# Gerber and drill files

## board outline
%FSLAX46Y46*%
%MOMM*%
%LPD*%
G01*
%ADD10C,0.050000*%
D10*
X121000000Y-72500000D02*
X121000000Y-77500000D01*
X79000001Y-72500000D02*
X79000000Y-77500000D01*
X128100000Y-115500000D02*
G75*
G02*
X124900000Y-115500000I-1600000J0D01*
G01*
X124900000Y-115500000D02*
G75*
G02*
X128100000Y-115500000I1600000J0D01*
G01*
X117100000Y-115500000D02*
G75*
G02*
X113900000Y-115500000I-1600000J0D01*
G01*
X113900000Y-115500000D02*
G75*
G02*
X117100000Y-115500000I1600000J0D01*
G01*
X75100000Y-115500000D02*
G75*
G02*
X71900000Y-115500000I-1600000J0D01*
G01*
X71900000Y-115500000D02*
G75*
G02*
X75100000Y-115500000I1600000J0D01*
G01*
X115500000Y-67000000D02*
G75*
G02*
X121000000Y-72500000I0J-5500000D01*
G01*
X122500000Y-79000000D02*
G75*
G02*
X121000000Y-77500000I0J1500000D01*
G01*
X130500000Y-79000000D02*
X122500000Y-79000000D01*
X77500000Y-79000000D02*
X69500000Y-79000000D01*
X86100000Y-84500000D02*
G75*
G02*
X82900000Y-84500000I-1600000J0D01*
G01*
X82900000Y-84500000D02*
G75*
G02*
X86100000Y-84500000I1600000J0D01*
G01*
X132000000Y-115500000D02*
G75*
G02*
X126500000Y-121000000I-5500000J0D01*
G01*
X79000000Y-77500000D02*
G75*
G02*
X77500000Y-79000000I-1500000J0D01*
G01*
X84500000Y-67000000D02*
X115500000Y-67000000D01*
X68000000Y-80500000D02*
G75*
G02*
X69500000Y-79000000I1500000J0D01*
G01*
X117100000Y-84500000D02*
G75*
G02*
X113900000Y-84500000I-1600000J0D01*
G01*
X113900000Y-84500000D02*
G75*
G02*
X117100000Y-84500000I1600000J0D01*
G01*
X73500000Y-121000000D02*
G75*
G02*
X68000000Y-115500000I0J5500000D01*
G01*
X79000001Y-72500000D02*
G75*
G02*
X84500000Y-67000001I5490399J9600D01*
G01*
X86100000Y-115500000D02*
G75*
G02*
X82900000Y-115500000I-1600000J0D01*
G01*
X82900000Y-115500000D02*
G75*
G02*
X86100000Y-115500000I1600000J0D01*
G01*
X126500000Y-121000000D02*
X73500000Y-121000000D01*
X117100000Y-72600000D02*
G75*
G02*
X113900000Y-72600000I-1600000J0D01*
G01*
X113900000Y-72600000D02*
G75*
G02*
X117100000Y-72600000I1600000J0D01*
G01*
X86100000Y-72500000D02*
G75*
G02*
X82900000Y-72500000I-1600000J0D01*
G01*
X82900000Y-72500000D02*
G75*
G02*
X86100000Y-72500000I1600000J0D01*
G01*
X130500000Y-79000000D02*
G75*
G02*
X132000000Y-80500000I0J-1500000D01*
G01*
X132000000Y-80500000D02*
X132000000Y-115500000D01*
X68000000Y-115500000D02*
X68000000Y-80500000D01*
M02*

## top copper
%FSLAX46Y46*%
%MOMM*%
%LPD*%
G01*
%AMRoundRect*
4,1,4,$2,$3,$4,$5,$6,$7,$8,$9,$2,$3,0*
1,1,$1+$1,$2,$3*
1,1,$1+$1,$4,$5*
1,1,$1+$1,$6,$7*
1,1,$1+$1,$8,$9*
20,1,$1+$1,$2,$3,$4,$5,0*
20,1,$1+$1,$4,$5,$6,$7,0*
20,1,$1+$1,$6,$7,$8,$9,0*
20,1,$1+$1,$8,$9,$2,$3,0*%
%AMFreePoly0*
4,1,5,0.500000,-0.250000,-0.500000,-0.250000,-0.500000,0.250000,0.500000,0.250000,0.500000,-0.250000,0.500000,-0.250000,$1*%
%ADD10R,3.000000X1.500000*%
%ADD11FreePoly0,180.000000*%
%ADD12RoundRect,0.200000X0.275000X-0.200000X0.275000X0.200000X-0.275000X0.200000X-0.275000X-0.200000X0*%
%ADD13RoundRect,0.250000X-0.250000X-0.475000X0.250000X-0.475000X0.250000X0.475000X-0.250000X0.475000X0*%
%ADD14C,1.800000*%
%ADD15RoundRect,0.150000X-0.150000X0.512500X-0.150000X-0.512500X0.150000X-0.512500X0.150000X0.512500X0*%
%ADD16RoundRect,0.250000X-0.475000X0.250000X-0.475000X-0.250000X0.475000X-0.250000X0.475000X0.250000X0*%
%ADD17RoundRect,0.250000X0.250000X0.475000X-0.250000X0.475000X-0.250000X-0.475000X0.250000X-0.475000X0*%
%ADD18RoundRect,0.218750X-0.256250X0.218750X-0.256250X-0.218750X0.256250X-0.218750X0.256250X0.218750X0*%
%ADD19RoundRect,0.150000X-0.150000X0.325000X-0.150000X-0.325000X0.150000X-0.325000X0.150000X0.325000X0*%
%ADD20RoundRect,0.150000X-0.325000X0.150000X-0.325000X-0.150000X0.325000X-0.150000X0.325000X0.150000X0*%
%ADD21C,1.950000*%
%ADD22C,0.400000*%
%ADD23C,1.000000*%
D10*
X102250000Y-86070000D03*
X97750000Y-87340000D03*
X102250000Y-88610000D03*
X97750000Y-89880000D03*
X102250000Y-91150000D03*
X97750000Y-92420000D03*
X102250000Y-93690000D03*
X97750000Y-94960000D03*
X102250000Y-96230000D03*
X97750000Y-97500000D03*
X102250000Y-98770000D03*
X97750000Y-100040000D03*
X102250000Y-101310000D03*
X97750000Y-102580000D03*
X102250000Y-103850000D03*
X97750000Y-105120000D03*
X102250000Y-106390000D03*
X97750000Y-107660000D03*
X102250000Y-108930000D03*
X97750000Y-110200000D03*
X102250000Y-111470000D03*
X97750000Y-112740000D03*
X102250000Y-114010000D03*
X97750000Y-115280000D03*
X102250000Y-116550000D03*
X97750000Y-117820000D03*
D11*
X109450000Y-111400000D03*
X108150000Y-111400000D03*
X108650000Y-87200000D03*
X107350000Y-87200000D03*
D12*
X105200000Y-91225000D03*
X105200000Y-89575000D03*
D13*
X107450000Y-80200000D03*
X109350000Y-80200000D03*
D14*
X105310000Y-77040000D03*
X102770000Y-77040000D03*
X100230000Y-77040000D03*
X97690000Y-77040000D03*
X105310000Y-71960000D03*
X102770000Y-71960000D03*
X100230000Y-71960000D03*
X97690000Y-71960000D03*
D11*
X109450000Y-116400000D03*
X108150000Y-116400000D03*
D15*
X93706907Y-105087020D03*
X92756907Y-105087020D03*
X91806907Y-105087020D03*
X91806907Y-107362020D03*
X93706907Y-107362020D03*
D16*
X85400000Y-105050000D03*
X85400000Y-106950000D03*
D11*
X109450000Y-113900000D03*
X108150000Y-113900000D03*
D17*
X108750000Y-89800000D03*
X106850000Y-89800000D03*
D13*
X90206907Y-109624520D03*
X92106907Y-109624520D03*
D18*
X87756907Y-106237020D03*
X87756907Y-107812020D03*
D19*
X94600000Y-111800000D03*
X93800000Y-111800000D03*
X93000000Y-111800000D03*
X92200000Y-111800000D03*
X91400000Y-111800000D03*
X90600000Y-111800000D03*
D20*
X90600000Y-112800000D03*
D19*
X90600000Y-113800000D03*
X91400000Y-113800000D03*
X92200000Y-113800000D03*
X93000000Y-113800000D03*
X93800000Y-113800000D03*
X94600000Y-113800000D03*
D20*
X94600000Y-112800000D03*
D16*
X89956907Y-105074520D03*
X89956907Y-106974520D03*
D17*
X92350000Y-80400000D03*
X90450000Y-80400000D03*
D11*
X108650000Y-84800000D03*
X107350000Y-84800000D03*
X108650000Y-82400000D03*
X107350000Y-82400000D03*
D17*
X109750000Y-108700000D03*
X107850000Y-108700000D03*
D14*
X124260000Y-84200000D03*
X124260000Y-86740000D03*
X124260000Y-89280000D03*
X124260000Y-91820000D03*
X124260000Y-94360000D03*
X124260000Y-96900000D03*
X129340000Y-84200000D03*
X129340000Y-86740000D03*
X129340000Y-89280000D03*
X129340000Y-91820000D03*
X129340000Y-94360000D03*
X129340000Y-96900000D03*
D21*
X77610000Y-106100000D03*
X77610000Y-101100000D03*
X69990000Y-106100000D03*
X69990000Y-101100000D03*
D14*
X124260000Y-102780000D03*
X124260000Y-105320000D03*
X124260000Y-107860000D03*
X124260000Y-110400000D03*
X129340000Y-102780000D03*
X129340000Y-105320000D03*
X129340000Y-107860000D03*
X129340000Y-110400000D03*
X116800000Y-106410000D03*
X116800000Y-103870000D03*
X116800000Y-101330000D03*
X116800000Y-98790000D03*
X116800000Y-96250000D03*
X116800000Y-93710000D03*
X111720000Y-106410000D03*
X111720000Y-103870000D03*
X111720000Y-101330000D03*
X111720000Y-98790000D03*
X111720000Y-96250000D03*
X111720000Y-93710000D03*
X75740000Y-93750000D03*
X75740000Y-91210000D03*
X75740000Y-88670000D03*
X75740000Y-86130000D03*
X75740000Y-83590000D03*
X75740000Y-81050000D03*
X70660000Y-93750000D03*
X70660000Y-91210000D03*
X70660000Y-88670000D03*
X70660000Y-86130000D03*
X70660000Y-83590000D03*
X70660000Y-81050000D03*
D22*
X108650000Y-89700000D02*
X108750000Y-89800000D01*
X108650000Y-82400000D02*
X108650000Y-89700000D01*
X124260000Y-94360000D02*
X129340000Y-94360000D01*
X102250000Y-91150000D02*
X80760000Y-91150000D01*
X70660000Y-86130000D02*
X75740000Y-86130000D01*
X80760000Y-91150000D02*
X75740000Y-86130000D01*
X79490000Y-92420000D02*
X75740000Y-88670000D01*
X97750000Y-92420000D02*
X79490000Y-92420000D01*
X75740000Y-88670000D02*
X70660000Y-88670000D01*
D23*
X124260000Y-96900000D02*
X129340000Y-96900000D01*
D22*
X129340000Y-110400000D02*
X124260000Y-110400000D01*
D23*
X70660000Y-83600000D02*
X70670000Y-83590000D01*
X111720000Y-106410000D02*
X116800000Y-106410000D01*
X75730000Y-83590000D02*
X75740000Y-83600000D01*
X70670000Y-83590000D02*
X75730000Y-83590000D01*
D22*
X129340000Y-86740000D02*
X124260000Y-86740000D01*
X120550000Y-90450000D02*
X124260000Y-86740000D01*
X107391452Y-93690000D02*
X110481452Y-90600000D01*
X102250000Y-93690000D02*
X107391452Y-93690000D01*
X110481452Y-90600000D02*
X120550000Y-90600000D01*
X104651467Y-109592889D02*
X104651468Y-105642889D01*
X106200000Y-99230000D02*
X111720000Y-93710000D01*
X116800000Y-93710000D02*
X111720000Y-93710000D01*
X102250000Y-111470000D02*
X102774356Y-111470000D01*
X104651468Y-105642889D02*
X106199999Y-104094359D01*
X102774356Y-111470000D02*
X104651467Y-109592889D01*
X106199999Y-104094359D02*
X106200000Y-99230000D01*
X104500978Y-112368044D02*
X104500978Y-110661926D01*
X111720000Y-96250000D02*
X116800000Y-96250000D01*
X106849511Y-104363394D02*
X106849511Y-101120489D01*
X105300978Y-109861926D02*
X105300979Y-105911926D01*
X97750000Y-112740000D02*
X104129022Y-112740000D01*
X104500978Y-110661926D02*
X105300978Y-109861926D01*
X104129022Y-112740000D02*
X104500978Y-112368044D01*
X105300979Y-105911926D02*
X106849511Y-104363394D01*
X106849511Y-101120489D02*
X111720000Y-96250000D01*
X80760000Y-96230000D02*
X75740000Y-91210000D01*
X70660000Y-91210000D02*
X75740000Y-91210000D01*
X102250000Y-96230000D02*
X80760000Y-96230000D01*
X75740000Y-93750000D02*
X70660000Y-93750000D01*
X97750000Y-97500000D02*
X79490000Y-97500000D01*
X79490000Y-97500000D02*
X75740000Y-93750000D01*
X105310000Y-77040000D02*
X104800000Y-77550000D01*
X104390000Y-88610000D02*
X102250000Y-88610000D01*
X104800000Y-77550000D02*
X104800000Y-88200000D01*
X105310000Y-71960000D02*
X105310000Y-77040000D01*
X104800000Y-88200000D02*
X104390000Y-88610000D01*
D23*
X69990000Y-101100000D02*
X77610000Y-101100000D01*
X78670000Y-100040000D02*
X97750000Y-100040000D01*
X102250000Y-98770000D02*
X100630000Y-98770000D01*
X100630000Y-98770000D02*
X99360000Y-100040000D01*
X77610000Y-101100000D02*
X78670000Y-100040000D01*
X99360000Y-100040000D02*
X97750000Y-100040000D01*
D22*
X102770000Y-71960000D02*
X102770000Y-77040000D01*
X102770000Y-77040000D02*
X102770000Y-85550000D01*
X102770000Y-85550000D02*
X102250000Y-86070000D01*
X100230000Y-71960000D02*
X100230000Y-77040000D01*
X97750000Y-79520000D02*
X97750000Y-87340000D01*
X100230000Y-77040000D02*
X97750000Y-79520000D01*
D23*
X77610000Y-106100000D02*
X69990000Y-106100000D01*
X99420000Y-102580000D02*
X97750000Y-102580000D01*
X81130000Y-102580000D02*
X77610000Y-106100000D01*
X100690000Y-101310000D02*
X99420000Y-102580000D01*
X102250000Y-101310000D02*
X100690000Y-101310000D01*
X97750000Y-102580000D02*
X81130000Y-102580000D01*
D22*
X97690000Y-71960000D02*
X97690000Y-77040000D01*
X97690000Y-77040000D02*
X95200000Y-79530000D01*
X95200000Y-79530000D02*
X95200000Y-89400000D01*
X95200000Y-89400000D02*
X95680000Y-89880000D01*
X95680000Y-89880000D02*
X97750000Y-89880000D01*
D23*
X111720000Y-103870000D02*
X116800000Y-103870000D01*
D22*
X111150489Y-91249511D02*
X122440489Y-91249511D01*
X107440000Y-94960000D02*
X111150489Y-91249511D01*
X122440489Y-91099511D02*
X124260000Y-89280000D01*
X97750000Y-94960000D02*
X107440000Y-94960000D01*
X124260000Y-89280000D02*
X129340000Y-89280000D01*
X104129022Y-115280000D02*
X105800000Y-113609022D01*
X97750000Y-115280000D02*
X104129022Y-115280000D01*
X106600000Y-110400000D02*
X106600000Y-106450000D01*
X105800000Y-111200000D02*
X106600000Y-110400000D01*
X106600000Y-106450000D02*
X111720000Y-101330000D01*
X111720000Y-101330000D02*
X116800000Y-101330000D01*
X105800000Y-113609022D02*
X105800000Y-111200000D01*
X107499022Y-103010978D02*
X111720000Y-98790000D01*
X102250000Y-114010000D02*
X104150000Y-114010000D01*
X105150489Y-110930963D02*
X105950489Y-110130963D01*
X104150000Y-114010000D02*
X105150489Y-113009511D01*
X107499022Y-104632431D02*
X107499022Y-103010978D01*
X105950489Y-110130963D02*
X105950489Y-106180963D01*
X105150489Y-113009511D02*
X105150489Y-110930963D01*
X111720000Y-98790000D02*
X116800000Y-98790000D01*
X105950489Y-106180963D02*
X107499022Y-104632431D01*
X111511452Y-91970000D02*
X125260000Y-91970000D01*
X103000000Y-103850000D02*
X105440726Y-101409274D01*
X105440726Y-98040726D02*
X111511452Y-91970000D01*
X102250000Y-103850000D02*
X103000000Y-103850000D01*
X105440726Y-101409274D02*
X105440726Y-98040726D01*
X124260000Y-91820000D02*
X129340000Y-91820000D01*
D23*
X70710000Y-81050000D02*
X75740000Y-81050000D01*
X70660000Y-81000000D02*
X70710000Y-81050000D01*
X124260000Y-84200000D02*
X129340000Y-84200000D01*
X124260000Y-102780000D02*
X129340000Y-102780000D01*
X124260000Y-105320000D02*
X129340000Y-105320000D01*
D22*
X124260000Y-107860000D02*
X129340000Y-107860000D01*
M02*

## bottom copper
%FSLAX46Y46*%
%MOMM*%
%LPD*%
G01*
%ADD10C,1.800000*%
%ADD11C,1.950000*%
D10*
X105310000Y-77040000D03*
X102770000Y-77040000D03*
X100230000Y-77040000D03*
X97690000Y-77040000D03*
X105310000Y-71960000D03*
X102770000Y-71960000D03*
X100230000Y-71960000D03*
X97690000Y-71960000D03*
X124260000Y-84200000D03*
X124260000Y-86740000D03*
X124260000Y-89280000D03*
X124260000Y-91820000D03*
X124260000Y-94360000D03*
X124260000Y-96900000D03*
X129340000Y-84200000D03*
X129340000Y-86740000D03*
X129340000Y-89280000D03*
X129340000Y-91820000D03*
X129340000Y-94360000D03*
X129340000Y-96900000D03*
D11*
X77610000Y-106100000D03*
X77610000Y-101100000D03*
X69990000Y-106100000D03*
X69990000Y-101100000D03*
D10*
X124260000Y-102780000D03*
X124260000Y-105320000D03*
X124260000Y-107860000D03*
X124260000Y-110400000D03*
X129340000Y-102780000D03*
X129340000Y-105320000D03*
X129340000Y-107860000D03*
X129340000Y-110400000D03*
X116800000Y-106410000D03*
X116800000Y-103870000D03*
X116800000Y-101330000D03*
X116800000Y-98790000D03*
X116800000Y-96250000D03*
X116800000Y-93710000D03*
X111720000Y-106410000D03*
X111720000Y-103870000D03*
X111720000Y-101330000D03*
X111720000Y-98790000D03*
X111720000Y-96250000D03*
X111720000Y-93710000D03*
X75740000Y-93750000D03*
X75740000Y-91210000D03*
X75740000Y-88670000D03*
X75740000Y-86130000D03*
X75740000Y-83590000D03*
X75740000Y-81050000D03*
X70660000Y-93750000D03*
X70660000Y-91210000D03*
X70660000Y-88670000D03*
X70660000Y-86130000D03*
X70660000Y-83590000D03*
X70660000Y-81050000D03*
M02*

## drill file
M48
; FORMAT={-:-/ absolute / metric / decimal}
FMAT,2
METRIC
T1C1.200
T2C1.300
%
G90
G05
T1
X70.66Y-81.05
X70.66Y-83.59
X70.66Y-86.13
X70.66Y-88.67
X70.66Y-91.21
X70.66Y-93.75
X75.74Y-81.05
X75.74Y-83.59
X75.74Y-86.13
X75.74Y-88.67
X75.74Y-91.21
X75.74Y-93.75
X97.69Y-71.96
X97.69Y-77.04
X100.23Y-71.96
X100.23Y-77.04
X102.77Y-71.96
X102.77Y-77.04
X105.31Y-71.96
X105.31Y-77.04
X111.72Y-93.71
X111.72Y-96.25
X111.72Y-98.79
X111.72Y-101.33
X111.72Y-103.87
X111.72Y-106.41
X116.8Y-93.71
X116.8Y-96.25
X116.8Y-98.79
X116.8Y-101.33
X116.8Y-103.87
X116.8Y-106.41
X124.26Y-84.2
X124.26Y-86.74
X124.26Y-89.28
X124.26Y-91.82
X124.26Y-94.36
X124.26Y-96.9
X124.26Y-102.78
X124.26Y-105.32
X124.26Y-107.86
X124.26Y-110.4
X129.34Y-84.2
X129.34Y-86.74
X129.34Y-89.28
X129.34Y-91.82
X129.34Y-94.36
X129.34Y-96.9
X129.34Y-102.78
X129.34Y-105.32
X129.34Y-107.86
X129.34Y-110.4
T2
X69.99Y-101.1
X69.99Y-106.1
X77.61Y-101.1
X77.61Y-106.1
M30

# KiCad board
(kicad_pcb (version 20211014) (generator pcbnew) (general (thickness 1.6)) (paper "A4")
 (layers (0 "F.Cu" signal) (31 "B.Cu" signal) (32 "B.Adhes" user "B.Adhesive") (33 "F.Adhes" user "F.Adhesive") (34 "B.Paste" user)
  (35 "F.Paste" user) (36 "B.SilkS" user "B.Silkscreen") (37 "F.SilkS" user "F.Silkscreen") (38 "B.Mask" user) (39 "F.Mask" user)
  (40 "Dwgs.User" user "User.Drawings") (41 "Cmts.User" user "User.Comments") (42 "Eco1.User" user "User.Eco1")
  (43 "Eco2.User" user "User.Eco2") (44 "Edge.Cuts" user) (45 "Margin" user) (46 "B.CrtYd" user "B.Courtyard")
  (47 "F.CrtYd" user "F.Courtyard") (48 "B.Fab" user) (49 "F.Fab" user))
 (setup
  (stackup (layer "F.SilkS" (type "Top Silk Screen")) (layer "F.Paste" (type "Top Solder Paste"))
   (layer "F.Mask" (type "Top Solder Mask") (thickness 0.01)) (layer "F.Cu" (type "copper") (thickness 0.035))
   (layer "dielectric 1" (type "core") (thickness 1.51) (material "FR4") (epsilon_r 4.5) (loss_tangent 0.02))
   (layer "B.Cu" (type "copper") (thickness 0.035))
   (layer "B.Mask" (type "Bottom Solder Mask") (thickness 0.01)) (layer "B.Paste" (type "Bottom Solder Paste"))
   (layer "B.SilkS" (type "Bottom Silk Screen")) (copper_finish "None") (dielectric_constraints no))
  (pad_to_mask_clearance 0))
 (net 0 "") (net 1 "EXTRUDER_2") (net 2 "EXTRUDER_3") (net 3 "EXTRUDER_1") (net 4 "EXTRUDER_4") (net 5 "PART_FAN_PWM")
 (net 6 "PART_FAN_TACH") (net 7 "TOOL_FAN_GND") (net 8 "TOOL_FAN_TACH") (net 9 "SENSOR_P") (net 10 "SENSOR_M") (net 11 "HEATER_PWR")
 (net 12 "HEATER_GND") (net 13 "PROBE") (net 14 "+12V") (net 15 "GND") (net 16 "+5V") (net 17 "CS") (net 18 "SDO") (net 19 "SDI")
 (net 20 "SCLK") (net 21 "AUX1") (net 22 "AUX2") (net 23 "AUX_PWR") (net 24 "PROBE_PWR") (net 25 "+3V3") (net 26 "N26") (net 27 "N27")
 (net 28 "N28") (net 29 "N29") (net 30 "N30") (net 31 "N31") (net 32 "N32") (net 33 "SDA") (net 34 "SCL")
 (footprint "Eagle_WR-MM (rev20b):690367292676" (layer "F.Cu") (at 100 101.945 90)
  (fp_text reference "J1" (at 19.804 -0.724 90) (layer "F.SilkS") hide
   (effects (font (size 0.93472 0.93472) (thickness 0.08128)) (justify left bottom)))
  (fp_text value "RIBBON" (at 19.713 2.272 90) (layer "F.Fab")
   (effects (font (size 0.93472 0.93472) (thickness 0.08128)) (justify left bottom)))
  (pad "1" smd rect (at 15.875 2.25 270) (size 1.5 3) (layers "F.Cu" "F.Paste" "F.Mask") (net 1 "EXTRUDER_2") (solder_mask_margin 0.1016))
  (pad "2" smd rect (at 14.605 -2.25 270) (size 1.5 3) (layers "F.Cu" "F.Paste" "F.Mask") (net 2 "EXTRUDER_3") (solder_mask_margin 0.1016))
  (pad "3" smd rect (at 13.335 2.25 270) (size 1.5 3) (layers "F.Cu" "F.Paste" "F.Mask") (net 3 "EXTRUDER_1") (solder_mask_margin 0.1016))
  (pad "4" smd rect (at 12.065 -2.25 270) (size 1.5 3) (layers "F.Cu" "F.Paste" "F.Mask") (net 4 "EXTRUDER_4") (solder_mask_margin 0.1016))
  (pad "5" smd rect (at 10.795 2.25 270) (size 1.5 3) (layers "F.Cu" "F.Paste" "F.Mask") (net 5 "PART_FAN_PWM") (solder_mask_margin 0.1016))
  (pad "6" smd rect (at 9.525 -2.25 270) (size 1.5 3) (layers "F.Cu" "F.Paste" "F.Mask") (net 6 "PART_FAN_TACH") (solder_mask_margin 0.1016))
  (pad "7" smd rect (at 8.255 2.25 270) (size 1.5 3) (layers "F.Cu" "F.Paste" "F.Mask") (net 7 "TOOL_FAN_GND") (solder_mask_margin 0.1016))
  (pad "8" smd rect (at 6.985 -2.25 270) (size 1.5 3) (layers "F.Cu" "F.Paste" "F.Mask") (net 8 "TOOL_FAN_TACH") (solder_mask_margin 0.1016))
  (pad "9" smd rect (at 5.715 2.25 270) (size 1.5 3) (layers "F.Cu" "F.Paste" "F.Mask") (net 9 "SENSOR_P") (solder_mask_margin 0.1016))
  (pad "10" smd rect (at 4.445 -2.25 270) (size 1.5 3) (layers "F.Cu" "F.Paste" "F.Mask") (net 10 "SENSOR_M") (solder_mask_margin 0.1016))
  (pad "11" smd rect (at 3.175 2.25 270) (size 1.5 3) (layers "F.Cu" "F.Paste" "F.Mask") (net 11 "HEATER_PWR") (solder_mask_margin 0.1016))
  (pad "12" smd rect (at 1.905 -2.25 270) (size 1.5 3) (layers "F.Cu" "F.Paste" "F.Mask") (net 11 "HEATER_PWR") (solder_mask_margin 0.1016))
  (pad "13" smd rect (at 0.635 2.25 270) (size 1.5 3) (layers "F.Cu" "F.Paste" "F.Mask") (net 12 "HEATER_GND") (solder_mask_margin 0.1016))
  (pad "14" smd rect (at -0.635 -2.25 270) (size 1.5 3) (layers "F.Cu" "F.Paste" "F.Mask") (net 12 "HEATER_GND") (solder_mask_margin 0.1016))
  (pad "15" smd rect (at -1.905 2.25 270) (size 1.5 3) (layers "F.Cu" "F.Paste" "F.Mask") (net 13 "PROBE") (solder_mask_margin 0.1016))
  (pad "16" smd rect (at -3.175 -2.25 270) (size 1.5 3) (layers "F.Cu" "F.Paste" "F.Mask") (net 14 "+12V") (solder_mask_margin 0.1016))
  (pad "17" smd rect (at -4.445 2.25 270) (size 1.5 3) (layers "F.Cu" "F.Paste" "F.Mask") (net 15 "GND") (solder_mask_margin 0.1016))
  (pad "18" smd rect (at -5.715 -2.25 270) (size 1.5 3) (layers "F.Cu" "F.Paste" "F.Mask") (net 14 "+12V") (solder_mask_margin 0.1016))
  (pad "19" smd rect (at -6.985 2.25 270) (size 1.5 3) (layers "F.Cu" "F.Paste" "F.Mask") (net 15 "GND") (solder_mask_margin 0.1016))
  (pad "20" smd rect (at -8.255 -2.25 270) (size 1.5 3) (layers "F.Cu" "F.Paste" "F.Mask") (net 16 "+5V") (solder_mask_margin 0.1016))
  (pad "21" smd rect (at -9.525 2.25 270) (size 1.5 3) (layers "F.Cu" "F.Paste" "F.Mask") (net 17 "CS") (solder_mask_margin 0.1016))
  (pad "22" smd rect (at -10.795 -2.25 270) (size 1.5 3) (layers "F.Cu" "F.Paste" "F.Mask") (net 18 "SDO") (solder_mask_margin 0.1016))
  (pad "23" smd rect (at -12.065 2.25 270) (size 1.5 3) (layers "F.Cu" "F.Paste" "F.Mask") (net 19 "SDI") (solder_mask_margin 0.1016))
  (pad "24" smd rect (at -13.335 -2.25 270) (size 1.5 3) (layers "F.Cu" "F.Paste" "F.Mask") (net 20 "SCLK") (solder_mask_margin 0.1016))
  (pad "25" smd rect (at -14.605 2.25 270) (size 1.5 3) (layers "F.Cu" "F.Paste" "F.Mask") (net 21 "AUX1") (solder_mask_margin 0.1016))
  (pad "26" smd rect (at -15.875 -2.25 270) (size 1.5 3) (layers "F.Cu" "F.Paste" "F.Mask") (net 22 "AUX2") (solder_mask_margin 0.1016)))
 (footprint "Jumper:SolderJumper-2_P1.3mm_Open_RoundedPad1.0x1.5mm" (layer "F.Cu") (at 108.8 111.4 180)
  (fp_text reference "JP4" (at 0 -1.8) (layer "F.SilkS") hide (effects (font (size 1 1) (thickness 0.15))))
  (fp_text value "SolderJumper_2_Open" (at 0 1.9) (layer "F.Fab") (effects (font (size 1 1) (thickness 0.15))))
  (pad "1" smd custom locked (at -0.65 0 180) (size 1 0.5) (layers "F.Cu" "F.Mask") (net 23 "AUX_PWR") (zone_connect 2)
   (options (clearance outline) (anchor rect)) (primitives))
  (pad "2" smd custom locked (at 0.65 0 180) (size 1 0.5) (layers "F.Cu" "F.Mask") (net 14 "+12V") (zone_connect 2)
   (options (clearance outline) (anchor rect)) (primitives)))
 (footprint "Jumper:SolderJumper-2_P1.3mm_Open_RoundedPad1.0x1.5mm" (layer "F.Cu") (at 108 87.2 180)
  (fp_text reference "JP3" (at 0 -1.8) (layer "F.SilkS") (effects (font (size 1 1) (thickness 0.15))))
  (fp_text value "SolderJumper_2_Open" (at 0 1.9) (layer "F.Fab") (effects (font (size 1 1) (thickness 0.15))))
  (pad "1" smd custom locked (at -0.65 0 180) (size 1 0.5) (layers "F.Cu" "F.Mask") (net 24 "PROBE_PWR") (zone_connect 2)
   (options (clearance outline) (anchor rect)) (primitives))
  (pad "2" smd custom locked (at 0.65 0 180) (size 1 0.5) (layers "F.Cu" "F.Mask") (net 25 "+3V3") (zone_connect 2)
   (options (clearance outline) (anchor rect)) (primitives)))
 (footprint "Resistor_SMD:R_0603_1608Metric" (layer "F.Cu") (at 105.2 90.4 90)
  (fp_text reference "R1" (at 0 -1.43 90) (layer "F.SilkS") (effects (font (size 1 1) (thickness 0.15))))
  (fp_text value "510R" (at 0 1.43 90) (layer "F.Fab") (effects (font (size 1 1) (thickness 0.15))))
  (pad "1" smd roundrect locked (at -0.825 0 90) (size 0.8 0.95) (layers "F.Cu" "F.Paste" "F.Mask") (roundrect_rratio 0.25)
   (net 5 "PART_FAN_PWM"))
  (pad "2" smd roundrect locked (at 0.825 0 90) (size 0.8 0.95) (layers "F.Cu" "F.Paste" "F.Mask") (roundrect_rratio 0.25) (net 15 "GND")))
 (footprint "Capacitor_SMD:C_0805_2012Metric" (layer "F.Cu") (at 108.4 80.2)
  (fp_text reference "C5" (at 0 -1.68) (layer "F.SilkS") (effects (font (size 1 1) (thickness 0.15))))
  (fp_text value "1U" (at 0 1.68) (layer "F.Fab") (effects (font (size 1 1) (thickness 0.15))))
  (pad "1" smd roundrect locked (at -0.95 0) (size 1 1.45) (layers "F.Cu" "F.Paste" "F.Mask") (roundrect_rratio 0.25) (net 15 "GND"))
  (pad "2" smd roundrect locked (at 0.95 0) (size 1 1.45) (layers "F.Cu" "F.Paste" "F.Mask") (roundrect_rratio 0.25) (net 14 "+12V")))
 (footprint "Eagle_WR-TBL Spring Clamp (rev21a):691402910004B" (layer "F.Cu") (at 101.5 74.5 180)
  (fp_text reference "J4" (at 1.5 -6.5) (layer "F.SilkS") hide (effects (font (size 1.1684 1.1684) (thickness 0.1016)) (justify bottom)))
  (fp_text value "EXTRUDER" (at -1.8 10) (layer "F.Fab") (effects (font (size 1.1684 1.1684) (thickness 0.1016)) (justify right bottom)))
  (pad "1" thru_hole circle (at -3.81 -2.54 180) (size 1.8 1.8) (drill 1.2) (layers *.Cu *.Mask) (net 3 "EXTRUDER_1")
   (solder_mask_margin 0.1016))
  (pad "2" thru_hole circle (at -1.27 -2.54 180) (size 1.8 1.8) (drill 1.2) (layers *.Cu *.Mask) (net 1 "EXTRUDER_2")
   (solder_mask_margin 0.1016))
  (pad "3" thru_hole circle (at 1.27 -2.54 180) (size 1.8 1.8) (drill 1.2) (layers *.Cu *.Mask) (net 2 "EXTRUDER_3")
   (solder_mask_margin 0.1016))
  (pad "4" thru_hole circle (at 3.81 -2.54 180) (size 1.8 1.8) (drill 1.2) (layers *.Cu *.Mask) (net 4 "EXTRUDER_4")
   (solder_mask_margin 0.1016))
  (pad "A1" thru_hole circle (at -3.81 2.54 180) (size 1.8 1.8) (drill 1.2) (layers *.Cu *.Mask) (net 3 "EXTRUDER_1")
   (solder_mask_margin 0.1016))
  (pad "A2" thru_hole circle (at -1.27 2.54 180) (size 1.8 1.8) (drill 1.2) (layers *.Cu *.Mask) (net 1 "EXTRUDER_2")
   (solder_mask_margin 0.1016))
  (pad "A3" thru_hole circle (at 1.27 2.54 180) (size 1.8 1.8) (drill 1.2) (layers *.Cu *.Mask) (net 2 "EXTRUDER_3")
   (solder_mask_margin 0.1016))
  (pad "A4" thru_hole circle (at 3.81 2.54 180) (size 1.8 1.8) (drill 1.2) (layers *.Cu *.Mask) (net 4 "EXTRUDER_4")
   (solder_mask_margin 0.1016)))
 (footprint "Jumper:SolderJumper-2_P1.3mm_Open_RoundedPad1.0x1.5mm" (layer "F.Cu") (at 108.8 116.4 180)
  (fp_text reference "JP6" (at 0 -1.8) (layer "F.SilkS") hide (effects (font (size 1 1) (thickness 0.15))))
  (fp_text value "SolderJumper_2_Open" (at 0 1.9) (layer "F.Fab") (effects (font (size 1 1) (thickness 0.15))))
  (pad "1" smd custom locked (at -0.65 0 180) (size 1 0.5) (layers "F.Cu" "F.Mask") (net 23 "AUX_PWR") (zone_connect 2)
   (options (clearance outline) (anchor rect)) (primitives))
  (pad "2" smd custom locked (at 0.65 0 180) (size 1 0.5) (layers "F.Cu" "F.Mask") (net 25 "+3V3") (zone_connect 2)
   (options (clearance outline) (anchor rect)) (primitives)))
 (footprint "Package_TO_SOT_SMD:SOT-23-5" (layer "F.Cu") (at 92.756907 106.22452 -90)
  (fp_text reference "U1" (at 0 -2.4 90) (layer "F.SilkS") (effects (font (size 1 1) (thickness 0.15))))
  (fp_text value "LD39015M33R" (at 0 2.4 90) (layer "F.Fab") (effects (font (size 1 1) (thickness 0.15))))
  (pad "1" smd roundrect locked (at -1.1375 -0.95 270) (size 1.325 0.6) (layers "F.Cu" "F.Paste" "F.Mask") (roundrect_rratio 0.25)
   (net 16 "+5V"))
  (pad "2" smd roundrect locked (at -1.1375 0 270) (size 1.325 0.6) (layers "F.Cu" "F.Paste" "F.Mask") (roundrect_rratio 0.25)
   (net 15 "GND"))
  (pad "3" smd roundrect locked (at -1.1375 0.95 270) (size 1.325 0.6) (layers "F.Cu" "F.Paste" "F.Mask") (roundrect_rratio 0.25)
   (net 16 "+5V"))
  (pad "4" smd roundrect locked (at 1.1375 0.95 270) (size 1.325 0.6) (layers "F.Cu" "F.Paste" "F.Mask") (roundrect_rratio 0.25)
   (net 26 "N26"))
  (pad "5" smd roundrect locked (at 1.1375 -0.95 270) (size 1.325 0.6) (layers "F.Cu" "F.Paste" "F.Mask") (roundrect_rratio 0.25)
   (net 25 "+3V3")))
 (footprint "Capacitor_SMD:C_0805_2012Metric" (layer "F.Cu") (at 85.4 106 -90)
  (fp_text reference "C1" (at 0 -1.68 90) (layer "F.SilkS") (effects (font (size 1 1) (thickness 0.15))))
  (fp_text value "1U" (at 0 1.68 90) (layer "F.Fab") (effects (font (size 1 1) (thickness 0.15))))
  (pad "1" smd roundrect locked (at -0.95 0 270) (size 1 1.45) (layers "F.Cu" "F.Paste" "F.Mask") (roundrect_rratio 0.25) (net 16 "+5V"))
  (pad "2" smd roundrect locked (at 0.95 0 270) (size 1 1.45) (layers "F.Cu" "F.Paste" "F.Mask") (roundrect_rratio 0.25) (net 15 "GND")))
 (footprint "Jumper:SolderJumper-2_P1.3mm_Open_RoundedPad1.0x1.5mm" (layer "F.Cu") (at 108.8 113.9 180)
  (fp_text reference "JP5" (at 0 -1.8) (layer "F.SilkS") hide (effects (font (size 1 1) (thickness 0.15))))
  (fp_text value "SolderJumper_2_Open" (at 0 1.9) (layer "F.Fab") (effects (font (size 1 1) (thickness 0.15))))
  (pad "1" smd custom locked (at -0.65 0 180) (size 1 0.5) (layers "F.Cu" "F.Mask") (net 23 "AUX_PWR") (zone_connect 2)
   (options (clearance outline) (anchor rect)) (primitives))
  (pad "2" smd custom locked (at 0.65 0 180) (size 1 0.5) (layers "F.Cu" "F.Mask") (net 16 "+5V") (zone_connect 2)
   (options (clearance outline) (anchor rect)) (primitives)))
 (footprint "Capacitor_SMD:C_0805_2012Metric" (layer "F.Cu") (at 107.8 89.8 180)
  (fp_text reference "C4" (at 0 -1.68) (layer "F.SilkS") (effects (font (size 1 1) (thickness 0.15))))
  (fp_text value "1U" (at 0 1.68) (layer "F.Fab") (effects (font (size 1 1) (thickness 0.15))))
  (pad "1" smd roundrect locked (at -0.95 0 180) (size 1 1.45) (layers "F.Cu" "F.Paste" "F.Mask") (roundrect_rratio 0.25)
   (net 24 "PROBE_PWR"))
  (pad "2" smd roundrect locked (at 0.95 0 180) (size 1 1.45) (layers "F.Cu" "F.Paste" "F.Mask") (roundrect_rratio 0.25) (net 15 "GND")))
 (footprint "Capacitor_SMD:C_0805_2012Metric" (layer "F.Cu") (at 91.156907 109.62452)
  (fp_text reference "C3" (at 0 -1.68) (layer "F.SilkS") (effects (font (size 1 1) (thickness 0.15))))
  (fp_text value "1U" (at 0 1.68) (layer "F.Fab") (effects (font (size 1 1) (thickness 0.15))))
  (pad "1" smd roundrect locked (at -0.95 0) (size 1 1.45) (layers "F.Cu" "F.Paste" "F.Mask") (roundrect_rratio 0.25) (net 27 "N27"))
  (pad "2" smd roundrect locked (at 0.95 0) (size 1 1.45) (layers "F.Cu" "F.Paste" "F.Mask") (roundrect_rratio 0.25) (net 15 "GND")))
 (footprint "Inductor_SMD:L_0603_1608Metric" (layer "F.Cu") (at 87.756907 107.02452 -90)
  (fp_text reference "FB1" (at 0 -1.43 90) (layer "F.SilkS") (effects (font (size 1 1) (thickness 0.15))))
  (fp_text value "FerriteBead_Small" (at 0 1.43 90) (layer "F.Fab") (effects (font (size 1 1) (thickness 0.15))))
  (pad "1" smd roundrect locked (at -0.7875 0 270) (size 0.875 0.95) (layers "F.Cu" "F.Paste" "F.Mask") (roundrect_rratio 0.25)
   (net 25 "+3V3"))
  (pad "2" smd roundrect locked (at 0.7875 0 270) (size 0.875 0.95) (layers "F.Cu" "F.Paste" "F.Mask") (roundrect_rratio 0.25)
   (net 27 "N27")))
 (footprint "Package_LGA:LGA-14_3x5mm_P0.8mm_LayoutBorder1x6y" (layer "F.Cu") (at 92.6 112.8 -90)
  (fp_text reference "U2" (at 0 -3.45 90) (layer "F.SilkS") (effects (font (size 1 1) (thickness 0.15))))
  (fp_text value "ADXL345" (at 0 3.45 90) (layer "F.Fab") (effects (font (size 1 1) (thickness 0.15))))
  (pad "1" smd roundrect locked (at -1 -2 270) (size 0.95 0.6) (layers "F.Cu" "F.Paste" "F.Mask") (roundrect_rratio 0.25) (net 25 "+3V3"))
  (pad "2" smd roundrect locked (at -1 -1.2 270) (size 0.95 0.6) (layers "F.Cu" "F.Paste" "F.Mask") (roundrect_rratio 0.25) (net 15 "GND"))
  (pad "3" smd roundrect locked (at -1 -0.4 270) (size 0.95 0.6) (layers "F.Cu" "F.Paste" "F.Mask") (roundrect_rratio 0.25) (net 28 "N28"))
  (pad "4" smd roundrect locked (at -1 0.4 270) (size 0.95 0.6) (layers "F.Cu" "F.Paste" "F.Mask") (roundrect_rratio 0.25) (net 15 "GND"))
  (pad "5" smd roundrect locked (at -1 1.2 270) (size 0.95 0.6) (layers "F.Cu" "F.Paste" "F.Mask") (roundrect_rratio 0.25) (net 15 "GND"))
  (pad "6" smd roundrect locked (at -1 2 270) (size 0.95 0.6) (layers "F.Cu" "F.Paste" "F.Mask") (roundrect_rratio 0.25) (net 27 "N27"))
  (pad "7" smd roundrect locked (at 0 2 270) (size 0.6 0.95) (layers "F.Cu" "F.Paste" "F.Mask") (roundrect_rratio 0.25) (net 17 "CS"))
  (pad "8" smd roundrect locked (at 1 2 270) (size 0.95 0.6) (layers "F.Cu" "F.Paste" "F.Mask") (roundrect_rratio 0.25) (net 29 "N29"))
  (pad "9" smd roundrect locked (at 1 1.2 270) (size 0.95 0.6) (layers "F.Cu" "F.Paste" "F.Mask") (roundrect_rratio 0.25) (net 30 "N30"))
  (pad "10" smd roundrect locked (at 1 0.4 270) (size 0.95 0.6) (layers "F.Cu" "F.Paste" "F.Mask") (roundrect_rratio 0.25) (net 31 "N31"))
  (pad "11" smd roundrect locked (at 1 -0.4 270) (size 0.95 0.6) (layers "F.Cu" "F.Paste" "F.Mask") (roundrect_rratio 0.25) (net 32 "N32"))
  (pad "12" smd roundrect locked (at 1 -1.2 270) (size 0.95 0.6) (layers "F.Cu" "F.Paste" "F.Mask") (roundrect_rratio 0.25) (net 18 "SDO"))
  (pad "13" smd roundrect locked (at 1 -2 270) (size 0.95 0.6) (layers "F.Cu" "F.Paste" "F.Mask") (roundrect_rratio 0.25) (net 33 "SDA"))
  (pad "14" smd roundrect locked (at 0 -2 270) (size 0.6 0.95) (layers "F.Cu" "F.Paste" "F.Mask") (roundrect_rratio 0.25) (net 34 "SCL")))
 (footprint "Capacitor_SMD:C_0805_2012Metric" (layer "F.Cu") (at 89.956907 106.02452 -90)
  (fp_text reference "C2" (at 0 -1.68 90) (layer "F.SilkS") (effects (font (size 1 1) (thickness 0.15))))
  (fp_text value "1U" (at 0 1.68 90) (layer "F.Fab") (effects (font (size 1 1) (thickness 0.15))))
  (pad "1" smd roundrect locked (at -0.95 0 270) (size 1 1.45) (layers "F.Cu" "F.Paste" "F.Mask") (roundrect_rratio 0.25) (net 25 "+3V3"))
  (pad "2" smd roundrect locked (at 0.95 0 270) (size 1 1.45) (layers "F.Cu" "F.Paste" "F.Mask") (roundrect_rratio 0.25) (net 15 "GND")))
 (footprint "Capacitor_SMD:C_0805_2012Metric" (layer "F.Cu") (at 91.4 80.4 180)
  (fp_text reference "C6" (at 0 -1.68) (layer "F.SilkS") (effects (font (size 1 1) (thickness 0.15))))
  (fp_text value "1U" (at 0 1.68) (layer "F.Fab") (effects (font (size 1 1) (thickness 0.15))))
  (pad "1" smd roundrect locked (at -0.95 0 180) (size 1 1.45) (layers "F.Cu" "F.Paste" "F.Mask") (roundrect_rratio 0.25) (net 15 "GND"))
  (pad "2" smd roundrect locked (at 0.95 0 180) (size 1 1.45) (layers "F.Cu" "F.Paste" "F.Mask") (roundrect_rratio 0.25) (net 14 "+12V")))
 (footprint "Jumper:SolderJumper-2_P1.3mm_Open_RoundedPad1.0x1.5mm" (layer "F.Cu") (at 108 84.8 180)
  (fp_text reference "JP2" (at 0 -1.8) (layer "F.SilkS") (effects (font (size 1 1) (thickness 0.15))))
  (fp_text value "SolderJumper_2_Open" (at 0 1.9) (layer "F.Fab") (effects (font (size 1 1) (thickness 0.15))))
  (pad "1" smd custom locked (at -0.65 0 180) (size 1 0.5) (layers "F.Cu" "F.Mask") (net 24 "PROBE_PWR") (zone_connect 2)
   (options (clearance outline) (anchor rect)) (primitives))
  (pad "2" smd custom locked (at 0.65 0 180) (size 1 0.5) (layers "F.Cu" "F.Mask") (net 16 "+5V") (zone_connect 2)
   (options (clearance outline) (anchor rect)) (primitives)))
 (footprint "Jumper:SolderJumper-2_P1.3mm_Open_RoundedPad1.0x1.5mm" (layer "F.Cu") (at 108 82.4 180)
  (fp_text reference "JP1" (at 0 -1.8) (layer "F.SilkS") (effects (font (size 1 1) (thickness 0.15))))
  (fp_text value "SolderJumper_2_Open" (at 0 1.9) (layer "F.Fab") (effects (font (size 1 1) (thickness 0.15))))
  (pad "1" smd custom locked (at -0.65 0 180) (size 1 0.5) (layers "F.Cu" "F.Mask") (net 24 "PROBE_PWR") (zone_connect 2)
   (options (clearance outline) (anchor rect)) (primitives))
  (pad "2" smd custom locked (at 0.65 0 180) (size 1 0.5) (layers "F.Cu" "F.Mask") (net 14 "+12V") (zone_connect 2)
   (options (clearance outline) (anchor rect)) (primitives)))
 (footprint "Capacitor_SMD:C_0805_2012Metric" (layer "F.Cu") (at 108.8 108.7 180)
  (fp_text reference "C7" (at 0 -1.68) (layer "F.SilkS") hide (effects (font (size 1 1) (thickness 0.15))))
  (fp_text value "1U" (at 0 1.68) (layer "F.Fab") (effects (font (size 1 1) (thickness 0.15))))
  (pad "1" smd roundrect locked (at -0.95 0 180) (size 1 1.45) (layers "F.Cu" "F.Paste" "F.Mask") (roundrect_rratio 0.25) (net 23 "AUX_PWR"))
  (pad "2" smd roundrect locked (at 0.95 0 180) (size 1 1.45) (layers "F.Cu" "F.Paste" "F.Mask") (roundrect_rratio 0.25) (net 15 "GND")))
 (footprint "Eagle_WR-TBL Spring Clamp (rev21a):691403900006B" (layer "B.Cu") (at 126.8 90.55 -90)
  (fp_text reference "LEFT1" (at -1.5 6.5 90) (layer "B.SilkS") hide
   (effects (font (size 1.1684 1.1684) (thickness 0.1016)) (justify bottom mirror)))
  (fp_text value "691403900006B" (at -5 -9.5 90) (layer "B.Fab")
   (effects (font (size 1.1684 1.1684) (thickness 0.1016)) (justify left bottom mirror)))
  (pad "1" thru_hole circle (at -6.35 2.54 270) (size 1.8 1.8) (drill 1.2) (layers *.Cu *.Mask) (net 14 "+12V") (solder_mask_margin 0.1016))
  (pad "2" thru_hole circle (at -3.81 2.54 270) (size 1.8 1.8) (drill 1.2) (layers *.Cu *.Mask) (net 7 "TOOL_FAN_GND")
   (solder_mask_margin 0.1016))
  (pad "3" thru_hole circle (at -1.27 2.54 270) (size 1.8 1.8) (drill 1.2) (layers *.Cu *.Mask) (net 8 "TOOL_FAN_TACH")
   (solder_mask_margin 0.1016))
  (pad "4" thru_hole circle (at 1.27 2.54 270) (size 1.8 1.8) (drill 1.2) (layers *.Cu *.Mask) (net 13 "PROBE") (solder_mask_margin 0.1016))
  (pad "5" thru_hole circle (at 3.81 2.54 270) (size 1.8 1.8) (drill 1.2) (layers *.Cu *.Mask) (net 24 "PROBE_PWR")
   (solder_mask_margin 0.1016))
  (pad "6" thru_hole circle (at 6.35 2.54 270) (size 1.8 1.8) (drill 1.2) (layers *.Cu *.Mask) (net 15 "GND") (solder_mask_margin 0.1016))
  (pad "A1" thru_hole circle (at -6.35 -2.54 270) (size 1.8 1.8) (drill 1.2) (layers *.Cu *.Mask) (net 14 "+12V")
   (solder_mask_margin 0.1016))
  (pad "A2" thru_hole circle (at -3.81 -2.54 270) (size 1.8 1.8) (drill 1.2) (layers *.Cu *.Mask) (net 7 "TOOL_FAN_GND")
   (solder_mask_margin 0.1016))
  (pad "A3" thru_hole circle (at -1.27 -2.54 270) (size 1.8 1.8) (drill 1.2) (layers *.Cu *.Mask) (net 8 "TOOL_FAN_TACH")
   (solder_mask_margin 0.1016))
  (pad "A4" thru_hole circle (at 1.27 -2.54 270) (size 1.8 1.8) (drill 1.2) (layers *.Cu *.Mask) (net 13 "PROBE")
   (solder_mask_margin 0.1016))
  (pad "A5" thru_hole circle (at 3.81 -2.54 270) (size 1.8 1.8) (drill 1.2) (layers *.Cu *.Mask) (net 24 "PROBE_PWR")
   (solder_mask_margin 0.1016))
  (pad "A6" thru_hole circle (at 6.35 -2.54 270) (size 1.8 1.8) (drill 1.2) (layers *.Cu *.Mask) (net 15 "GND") (solder_mask_margin 0.1016)))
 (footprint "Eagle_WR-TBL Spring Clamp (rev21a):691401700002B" (layer "B.Cu") (at 73.8 103.6 90)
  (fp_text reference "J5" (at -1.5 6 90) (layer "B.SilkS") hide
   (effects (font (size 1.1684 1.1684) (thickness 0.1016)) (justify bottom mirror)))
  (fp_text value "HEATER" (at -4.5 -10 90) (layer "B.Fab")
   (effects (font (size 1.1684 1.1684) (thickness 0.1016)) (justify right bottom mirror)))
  (pad "1" thru_hole circle (at -2.5 3.81 90) (size 1.95 1.95) (drill 1.3) (layers *.Cu *.Mask) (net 12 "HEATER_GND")
   (solder_mask_margin 0.1016))
  (pad "2" thru_hole circle (at 2.5 3.81 90) (size 1.95 1.95) (drill 1.3) (layers *.Cu *.Mask) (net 11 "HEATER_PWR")
   (solder_mask_margin 0.1016))
  (pad "A1" thru_hole circle (at -2.5 -3.81 90) (size 1.95 1.95) (drill 1.3) (layers *.Cu *.Mask) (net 12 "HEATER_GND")
   (solder_mask_margin 0.1016))
  (pad "A2" thru_hole circle (at 2.5 -3.81 90) (size 1.95 1.95) (drill 1.3) (layers *.Cu *.Mask) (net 11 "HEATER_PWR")
   (solder_mask_margin 0.1016)))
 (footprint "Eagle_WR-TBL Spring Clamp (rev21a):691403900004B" (layer "B.Cu") (at 126.8 106.59 -90)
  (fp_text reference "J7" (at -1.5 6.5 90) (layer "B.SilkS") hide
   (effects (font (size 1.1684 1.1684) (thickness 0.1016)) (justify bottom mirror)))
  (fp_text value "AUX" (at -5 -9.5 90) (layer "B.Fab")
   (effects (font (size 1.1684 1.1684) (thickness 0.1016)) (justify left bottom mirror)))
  (pad "1" thru_hole circle (at -3.81 2.54 270) (size 1.8 1.8) (drill 1.2) (layers *.Cu *.Mask) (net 21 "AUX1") (solder_mask_margin 0.1016))
  (pad "2" thru_hole circle (at -1.27 2.54 270) (size 1.8 1.8) (drill 1.2) (layers *.Cu *.Mask) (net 22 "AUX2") (solder_mask_margin 0.1016))
  (pad "3" thru_hole circle (at 1.27 2.54 270) (size 1.8 1.8) (drill 1.2) (layers *.Cu *.Mask) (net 23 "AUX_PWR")
   (solder_mask_margin 0.1016))
  (pad "4" thru_hole circle (at 3.81 2.54 270) (size 1.8 1.8) (drill 1.2) (layers *.Cu *.Mask) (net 15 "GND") (solder_mask_margin 0.1016))
  (pad "A1" thru_hole circle (at -3.81 -2.54 270) (size 1.8 1.8) (drill 1.2) (layers *.Cu *.Mask) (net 21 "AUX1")
   (solder_mask_margin 0.1016))
  (pad "A2" thru_hole circle (at -1.27 -2.54 270) (size 1.8 1.8) (drill 1.2) (layers *.Cu *.Mask) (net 22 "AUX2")
   (solder_mask_margin 0.1016))
  (pad "A3" thru_hole circle (at 1.27 -2.54 270) (size 1.8 1.8) (drill 1.2) (layers *.Cu *.Mask) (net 23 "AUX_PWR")
   (solder_mask_margin 0.1016))
  (pad "A4" thru_hole circle (at 3.81 -2.54 270) (size 1.8 1.8) (drill 1.2) (layers *.Cu *.Mask) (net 15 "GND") (solder_mask_margin 0.1016)))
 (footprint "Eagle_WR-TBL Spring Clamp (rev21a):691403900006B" (layer "B.Cu") (at 114.26 100.06 90)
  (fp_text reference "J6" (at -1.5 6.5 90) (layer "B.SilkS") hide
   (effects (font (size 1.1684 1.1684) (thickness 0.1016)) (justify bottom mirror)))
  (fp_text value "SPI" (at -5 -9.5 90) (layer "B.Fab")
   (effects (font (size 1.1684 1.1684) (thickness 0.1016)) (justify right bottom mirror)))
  (pad "1" thru_hole circle (at -6.35 2.54 90) (size 1.8 1.8) (drill 1.2) (layers *.Cu *.Mask) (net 15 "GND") (solder_mask_margin 0.1016))
  (pad "2" thru_hole circle (at -3.81 2.54 90) (size 1.8 1.8) (drill 1.2) (layers *.Cu *.Mask) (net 16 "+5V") (solder_mask_margin 0.1016))
  (pad "3" thru_hole circle (at -1.27 2.54 90) (size 1.8 1.8) (drill 1.2) (layers *.Cu *.Mask) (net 20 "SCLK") (solder_mask_margin 0.1016))
  (pad "4" thru_hole circle (at 1.27 2.54 90) (size 1.8 1.8) (drill 1.2) (layers *.Cu *.Mask) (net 19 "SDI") (solder_mask_margin 0.1016))
  (pad "5" thru_hole circle (at 3.81 2.54 90) (size 1.8 1.8) (drill 1.2) (layers *.Cu *.Mask) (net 18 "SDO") (solder_mask_margin 0.1016))
  (pad "6" thru_hole circle (at 6.35 2.54 90) (size 1.8 1.8) (drill 1.2) (layers *.Cu *.Mask) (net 17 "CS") (solder_mask_margin 0.1016))
  (pad "A1" thru_hole circle (at -6.35 -2.54 90) (size 1.8 1.8) (drill 1.2) (layers *.Cu *.Mask) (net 15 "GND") (solder_mask_margin 0.1016))
  (pad "A2" thru_hole circle (at -3.81 -2.54 90) (size 1.8 1.8) (drill 1.2) (layers *.Cu *.Mask) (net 16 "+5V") (solder_mask_margin 0.1016))
  (pad "A3" thru_hole circle (at -1.27 -2.54 90) (size 1.8 1.8) (drill 1.2) (layers *.Cu *.Mask) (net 20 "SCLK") (solder_mask_margin 0.1016))
  (pad "A4" thru_hole circle (at 1.27 -2.54 90) (size 1.8 1.8) (drill 1.2) (layers *.Cu *.Mask) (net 19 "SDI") (solder_mask_margin 0.1016))
  (pad "A5" thru_hole circle (at 3.81 -2.54 90) (size 1.8 1.8) (drill 1.2) (layers *.Cu *.Mask) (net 18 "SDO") (solder_mask_margin 0.1016))
  (pad "A6" thru_hole circle (at 6.35 -2.54 90) (size 1.8 1.8) (drill 1.2) (layers *.Cu *.Mask) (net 17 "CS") (solder_mask_margin 0.1016)))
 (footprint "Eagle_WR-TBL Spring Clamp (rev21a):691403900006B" (layer "B.Cu") (at 73.2 87.4 90)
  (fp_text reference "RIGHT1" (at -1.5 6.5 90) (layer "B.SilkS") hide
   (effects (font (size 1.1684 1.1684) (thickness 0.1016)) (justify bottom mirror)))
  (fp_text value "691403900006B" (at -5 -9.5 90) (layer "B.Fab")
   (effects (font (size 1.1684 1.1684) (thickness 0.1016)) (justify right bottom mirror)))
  (pad "1" thru_hole circle (at -6.35 2.54 90) (size 1.8 1.8) (drill 1.2) (layers *.Cu *.Mask) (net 10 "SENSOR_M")
   (solder_mask_margin 0.1016))
  (pad "2" thru_hole circle (at -3.81 2.54 90) (size 1.8 1.8) (drill 1.2) (layers *.Cu *.Mask) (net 9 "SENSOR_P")
   (solder_mask_margin 0.1016))
  (pad "3" thru_hole circle (at -1.27 2.54 90) (size 1.8 1.8) (drill 1.2) (layers *.Cu *.Mask) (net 6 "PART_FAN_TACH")
   (solder_mask_margin 0.1016))
  (pad "4" thru_hole circle (at 1.27 2.54 90) (size 1.8 1.8) (drill 1.2) (layers *.Cu *.Mask) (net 5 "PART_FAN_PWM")
   (solder_mask_margin 0.1016))
  (pad "5" thru_hole circle (at 3.81 2.54 90) (size 1.8 1.8) (drill 1.2) (layers *.Cu *.Mask) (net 15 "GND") (solder_mask_margin 0.1016))
  (pad "6" thru_hole circle (at 6.35 2.54 90) (size 1.8 1.8) (drill 1.2) (layers *.Cu *.Mask) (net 14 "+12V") (solder_mask_margin 0.1016))
  (pad "A1" thru_hole circle (at -6.35 -2.54 90) (size 1.8 1.8) (drill 1.2) (layers *.Cu *.Mask) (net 10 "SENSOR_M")
   (solder_mask_margin 0.1016))
  (pad "A2" thru_hole circle (at -3.81 -2.54 90) (size 1.8 1.8) (drill 1.2) (layers *.Cu *.Mask) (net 9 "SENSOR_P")
   (solder_mask_margin 0.1016))
  (pad "A3" thru_hole circle (at -1.27 -2.54 90) (size 1.8 1.8) (drill 1.2) (layers *.Cu *.Mask) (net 6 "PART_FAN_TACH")
   (solder_mask_margin 0.1016))
  (pad "A4" thru_hole circle (at 1.27 -2.54 90) (size 1.8 1.8) (drill 1.2) (layers *.Cu *.Mask) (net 5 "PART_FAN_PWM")
   (solder_mask_margin 0.1016))
  (pad "A5" thru_hole circle (at 3.81 -2.54 90) (size 1.8 1.8) (drill 1.2) (layers *.Cu *.Mask) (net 15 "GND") (solder_mask_margin 0.1016))
  (pad "A6" thru_hole circle (at 6.35 -2.54 90) (size 1.8 1.8) (drill 1.2) (layers *.Cu *.Mask) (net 14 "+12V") (solder_mask_margin 0.1016)))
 (gr_line (start 121 72.5) (end 121 77.5) (layer "Edge.Cuts") (width 0.05))
 (gr_line (start 79.000001 72.5) (end 79 77.5) (layer "Edge.Cuts") (width 0.05))
 (gr_circle (center 126.5 115.5) (end 128.1 115.5) (layer "Edge.Cuts") (width 0.05) (fill none))
 (gr_circle (center 115.5 115.5) (end 117.1 115.5) (layer "Edge.Cuts") (width 0.05) (fill none))
 (gr_circle (center 73.5 115.5) (end 75.1 115.5) (layer "Edge.Cuts") (width 0.05) (fill none))
 (gr_arc (start 115.5 67) (mid 119.389087 68.610913) (end 121 72.5) (layer "Edge.Cuts") (width 0.05))
 (gr_arc (start 122.5 79) (mid 121.43934 78.56066) (end 121 77.5) (layer "Edge.Cuts") (width 0.05))
 (gr_line (start 130.5 79) (end 122.5 79) (layer "Edge.Cuts") (width 0.05))
 (gr_line (start 77.5 79) (end 69.5 79) (layer "Edge.Cuts") (width 0.05))
 (gr_circle (center 84.5 84.5) (end 86.1 84.5) (layer "Edge.Cuts") (width 0.05) (fill none))
 (gr_arc (start 132 115.5) (mid 130.389087 119.389087) (end 126.5 121) (layer "Edge.Cuts") (width 0.05))
 (gr_arc (start 79 77.5) (mid 78.56066 78.56066) (end 77.5 79) (layer "Edge.Cuts") (width 0.05))
 (gr_line (start 84.5 67) (end 115.5 67) (layer "Edge.Cuts") (width 0.05))
 (gr_arc (start 68 80.5) (mid 68.43934 79.43934) (end 69.5 79) (layer "Edge.Cuts") (width 0.05))
 (gr_circle (center 115.5 84.5) (end 117.1 84.5) (layer "Edge.Cuts") (width 0.05) (fill none))
 (gr_arc (start 73.5 121) (mid 69.610913 119.389087) (end 68 115.5) (layer "Edge.Cuts") (width 0.05))
 (gr_arc (start 79.000001 72.5) (mid 80.608101 68.608101) (end 84.5 67) (layer "Edge.Cuts") (width 0.05))
 (gr_circle (center 84.5 115.5) (end 86.1 115.5) (layer "Edge.Cuts") (width 0.05) (fill none))
 (gr_line (start 126.5 121) (end 73.5 121) (layer "Edge.Cuts") (width 0.05))
 (gr_circle (center 115.5 72.6) (end 117.1 72.6) (layer "Edge.Cuts") (width 0.05) (fill none))
 (gr_circle (center 84.5 72.5) (end 86.1 72.5) (layer "Edge.Cuts") (width 0.05) (fill none))
 (gr_arc (start 130.5 79) (mid 131.560659 79.43934) (end 132 80.5) (layer "Edge.Cuts") (width 0.05))
 (gr_line (start 132 80.5) (end 132 115.5) (layer "Edge.Cuts") (width 0.05))
 (gr_line (start 68 115.5) (end 68 80.5) (layer "Edge.Cuts") (width 0.05))
 (segment (start 108.65 89.7) (end 108.75 89.8) (width 0.4) (layer "F.Cu") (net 24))
 (segment (start 108.65 82.4) (end 108.65 89.7) (width 0.4) (layer "F.Cu") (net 24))
 (segment (start 124.26 94.36) (end 129.34 94.36) (width 0.4) (layer "F.Cu") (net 24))
 (segment (start 102.25 91.15) (end 80.76 91.15) (width 0.4) (layer "F.Cu") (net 5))
 (segment (start 70.66 86.13) (end 75.74 86.13) (width 0.4) (layer "F.Cu") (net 5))
 (segment (start 80.76 91.15) (end 75.74 86.13) (width 0.4) (layer "F.Cu") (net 5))
 (segment (start 79.49 92.42) (end 75.74 88.67) (width 0.4) (layer "F.Cu") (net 6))
 (segment (start 97.75 92.42) (end 79.49 92.42) (width 0.4) (layer "F.Cu") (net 6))
 (segment (start 75.74 88.67) (end 70.66 88.67) (width 0.4) (layer "F.Cu") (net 6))
 (segment (start 124.26 96.9) (end 129.34 96.9) (width 1) (layer "F.Cu") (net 15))
 (segment (start 129.34 110.4) (end 124.26 110.4) (width 0.4) (layer "F.Cu") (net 15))
 (segment (start 70.66 83.6) (end 70.67 83.59) (width 1) (layer "F.Cu") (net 15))
 (segment (start 111.72 106.41) (end 116.8 106.41) (width 1) (layer "F.Cu") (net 15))
 (segment (start 75.73 83.59) (end 75.74 83.6) (width 1) (layer "F.Cu") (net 15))
 (segment (start 70.67 83.59) (end 75.73 83.59) (width 1) (layer "F.Cu") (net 15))
 (segment (start 129.34 86.74) (end 124.26 86.74) (width 0.4) (layer "F.Cu") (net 7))
 (segment (start 120.55 90.45) (end 124.26 86.74) (width 0.4) (layer "F.Cu") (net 7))
 (segment (start 107.391452 93.69) (end 110.481452 90.6) (width 0.4) (layer "F.Cu") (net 7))
 (segment (start 102.25 93.69) (end 107.391452 93.69) (width 0.4) (layer "F.Cu") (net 7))
 (segment (start 110.481452 90.6) (end 120.55 90.6) (width 0.4) (layer "F.Cu") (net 7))
 (segment (start 104.651467 109.592889) (end 104.651468 105.642889) (width 0.4) (layer "F.Cu") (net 17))
 (segment (start 106.2 99.23) (end 111.72 93.71) (width 0.4) (layer "F.Cu") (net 17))
 (segment (start 116.8 93.71) (end 111.72 93.71) (width 0.4) (layer "F.Cu") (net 17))
 (segment (start 102.25 111.47) (end 102.774356 111.47) (width 0.4) (layer "F.Cu") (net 17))
 (segment (start 104.651468 105.642889) (end 106.199999 104.094359) (width 0.4) (layer "F.Cu") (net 17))
 (segment (start 102.774356 111.47) (end 104.651467 109.592889) (width 0.4) (layer "F.Cu") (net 17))
 (segment (start 106.199999 104.094359) (end 106.2 99.23) (width 0.4) (layer "F.Cu") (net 17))
 (segment (start 104.500978 112.368044) (end 104.500978 110.661926) (width 0.4) (layer "F.Cu") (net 18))
 (segment (start 111.72 96.25) (end 116.8 96.25) (width 0.4) (layer "F.Cu") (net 18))
 (segment (start 106.849511 104.363394) (end 106.849511 101.120489) (width 0.4) (layer "F.Cu") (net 18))
 (segment (start 105.300978 109.861926) (end 105.300979 105.911926) (width 0.4) (layer "F.Cu") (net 18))
 (segment (start 97.75 112.74) (end 104.129022 112.74) (width 0.4) (layer "F.Cu") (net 18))
 (segment (start 104.500978 110.661926) (end 105.300978 109.861926) (width 0.4) (layer "F.Cu") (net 18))
 (segment (start 104.129022 112.74) (end 104.500978 112.368044) (width 0.4) (layer "F.Cu") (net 18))
 (segment (start 105.300979 105.911926) (end 106.849511 104.363394) (width 0.4) (layer "F.Cu") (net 18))
 (segment (start 106.849511 101.120489) (end 111.72 96.25) (width 0.4) (layer "F.Cu") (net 18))
 (segment (start 80.76 96.23) (end 75.74 91.21) (width 0.4) (layer "F.Cu") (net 9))
 (segment (start 70.66 91.21) (end 75.74 91.21) (width 0.4) (layer "F.Cu") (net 9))
 (segment (start 102.25 96.23) (end 80.76 96.23) (width 0.4) (layer "F.Cu") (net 9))
 (segment (start 75.74 93.75) (end 70.66 93.75) (width 0.4) (layer "F.Cu") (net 10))
 (segment (start 97.75 97.5) (end 79.49 97.5) (width 0.4) (layer "F.Cu") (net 10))
 (segment (start 79.49 97.5) (end 75.74 93.75) (width 0.4) (layer "F.Cu") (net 10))
 (segment (start 105.31 77.04) (end 104.8 77.55) (width 0.4) (layer "F.Cu") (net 3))
 (segment (start 104.39 88.61) (end 102.25 88.61) (width 0.4) (layer "F.Cu") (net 3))
 (segment (start 104.8 77.55) (end 104.8 88.2) (width 0.4) (layer "F.Cu") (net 3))
 (segment (start 105.31 71.96) (end 105.31 77.04) (width 0.4) (layer "F.Cu") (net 3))
 (segment (start 104.8 88.2) (end 104.39 88.61) (width 0.4) (layer "F.Cu") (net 3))
 (segment (start 69.99 101.1) (end 77.61 101.1) (width 1) (layer "F.Cu") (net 11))
 (segment (start 78.67 100.04) (end 97.75 100.04) (width 1) (layer "F.Cu") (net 11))
 (segment (start 102.25 98.77) (end 100.63 98.77) (width 1) (layer "F.Cu") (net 11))
 (segment (start 100.63 98.77) (end 99.36 100.04) (width 1) (layer "F.Cu") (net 11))
 (segment (start 77.61 101.1) (end 78.67 100.04) (width 1) (layer "F.Cu") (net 11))
 (segment (start 99.36 100.04) (end 97.75 100.04) (width 1) (layer "F.Cu") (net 11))
 (segment (start 102.77 71.96) (end 102.77 77.04) (width 0.4) (layer "F.Cu") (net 1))
 (segment (start 102.77 77.04) (end 102.77 85.55) (width 0.4) (layer "F.Cu") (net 1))
 (segment (start 102.77 85.55) (end 102.25 86.07) (width 0.4) (layer "F.Cu") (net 1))
 (segment (start 100.23 71.96) (end 100.23 77.04) (width 0.4) (layer "F.Cu") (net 2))
 (segment (start 97.75 79.52) (end 97.75 87.34) (width 0.4) (layer "F.Cu") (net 2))
 (segment (start 100.23 77.04) (end 97.75 79.52) (width 0.4) (layer "F.Cu") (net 2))
 (segment (start 77.61 106.1) (end 69.99 106.1) (width 1) (layer "F.Cu") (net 12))
 (segment (start 99.42 102.58) (end 97.75 102.58) (width 1) (layer "F.Cu") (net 12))
 (segment (start 81.13 102.58) (end 77.61 106.1) (width 1) (layer "F.Cu") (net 12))
 (segment (start 100.69 101.31) (end 99.42 102.58) (width 1) (layer "F.Cu") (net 12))
 (segment (start 102.25 101.31) (end 100.69 101.31) (width 1) (layer "F.Cu") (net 12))
 (segment (start 97.75 102.58) (end 81.13 102.58) (width 1) (layer "F.Cu") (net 12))
 (segment (start 97.69 71.96) (end 97.69 77.04) (width 0.4) (layer "F.Cu") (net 4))
 (segment (start 97.69 77.04) (end 95.2 79.53) (width 0.4) (layer "F.Cu") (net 4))
 (segment (start 95.2 79.53) (end 95.2 89.4) (width 0.4) (layer "F.Cu") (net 4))
 (segment (start 95.2 89.4) (end 95.68 89.88) (width 0.4) (layer "F.Cu") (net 4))
 (segment (start 95.68 89.88) (end 97.75 89.88) (width 0.4) (layer "F.Cu") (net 4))
 (segment (start 111.72 103.87) (end 116.8 103.87) (width 1) (layer "F.Cu") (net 16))
 (segment (start 111.150489 91.249511) (end 122.440489 91.249511) (width 0.4) (layer "F.Cu") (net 8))
 (segment (start 107.44 94.96) (end 111.150489 91.249511) (width 0.4) (layer "F.Cu") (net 8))
 (segment (start 122.440489 91.099511) (end 124.26 89.28) (width 0.4) (layer "F.Cu") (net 8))
 (segment (start 97.75 94.96) (end 107.44 94.96) (width 0.4) (layer "F.Cu") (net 8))
 (segment (start 124.26 89.28) (end 129.34 89.28) (width 0.4) (layer "F.Cu") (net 8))
 (segment (start 104.129022 115.28) (end 105.8 113.609022) (width 0.4) (layer "F.Cu") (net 20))
 (segment (start 97.75 115.28) (end 104.129022 115.28) (width 0.4) (layer "F.Cu") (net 20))
 (segment (start 106.6 110.4) (end 106.6 106.45) (width 0.4) (layer "F.Cu") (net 20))
 (segment (start 105.8 111.2) (end 106.6 110.4) (width 0.4) (layer "F.Cu") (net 20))
 (segment (start 106.6 106.45) (end 111.72 101.33) (width 0.4) (layer "F.Cu") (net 20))
 (segment (start 111.72 101.33) (end 116.8 101.33) (width 0.4) (layer "F.Cu") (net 20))
 (segment (start 105.8 113.609022) (end 105.8 111.2) (width 0.4) (layer "F.Cu") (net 20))
 (segment (start 107.499022 103.010978) (end 111.72 98.79) (width 0.4) (layer "F.Cu") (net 19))
 (segment (start 102.25 114.01) (end 104.15 114.01) (width 0.4) (layer "F.Cu") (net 19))
 (segment (start 105.150489 110.930963) (end 105.950489 110.130963) (width 0.4) (layer "F.Cu") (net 19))
 (segment (start 104.15 114.01) (end 105.150489 113.009511) (width 0.4) (layer "F.Cu") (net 19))
 (segment (start 107.499022 104.632431) (end 107.499022 103.010978) (width 0.4) (layer "F.Cu") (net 19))
 (segment (start 105.950489 110.130963) (end 105.950489 106.180963) (width 0.4) (layer "F.Cu") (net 19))
 (segment (start 105.150489 113.009511) (end 105.150489 110.930963) (width 0.4) (layer "F.Cu") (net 19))
 (segment (start 111.72 98.79) (end 116.8 98.79) (width 0.4) (layer "F.Cu") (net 19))
 (segment (start 105.950489 106.180963) (end 107.499022 104.632431) (width 0.4) (layer "F.Cu") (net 19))
 (segment (start 111.511452 91.97) (end 125.26 91.97) (width 0.4) (layer "F.Cu") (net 13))
 (segment (start 103 103.85) (end 105.440726 101.409274) (width 0.4) (layer "F.Cu") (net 13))
 (segment (start 105.440726 98.040726) (end 111.511452 91.97) (width 0.4) (layer "F.Cu") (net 13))
 (segment (start 102.25 103.85) (end 103 103.85) (width 0.4) (layer "F.Cu") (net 13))
 (segment (start 105.440726 101.409274) (end 105.440726 98.040726) (width 0.4) (layer "F.Cu") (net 13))
 (segment (start 124.26 91.82) (end 129.34 91.82) (width 0.4) (layer "F.Cu") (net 13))
 (segment (start 70.71 81.05) (end 75.74 81.05) (width 1) (layer "F.Cu") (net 14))
 (segment (start 70.66 81) (end 70.71 81.05) (width 1) (layer "F.Cu") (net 14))
 (segment (start 124.26 84.2) (end 129.34 84.2) (width 1) (layer "F.Cu") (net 14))
 (segment (start 124.26 102.78) (end 129.34 102.78) (width 1) (layer "F.Cu") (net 21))
 (segment (start 124.26 105.32) (end 129.34 105.32) (width 1) (layer "F.Cu") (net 22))
 (segment (start 124.26 107.86) (end 129.34 107.86) (width 0.4) (layer "F.Cu") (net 23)))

